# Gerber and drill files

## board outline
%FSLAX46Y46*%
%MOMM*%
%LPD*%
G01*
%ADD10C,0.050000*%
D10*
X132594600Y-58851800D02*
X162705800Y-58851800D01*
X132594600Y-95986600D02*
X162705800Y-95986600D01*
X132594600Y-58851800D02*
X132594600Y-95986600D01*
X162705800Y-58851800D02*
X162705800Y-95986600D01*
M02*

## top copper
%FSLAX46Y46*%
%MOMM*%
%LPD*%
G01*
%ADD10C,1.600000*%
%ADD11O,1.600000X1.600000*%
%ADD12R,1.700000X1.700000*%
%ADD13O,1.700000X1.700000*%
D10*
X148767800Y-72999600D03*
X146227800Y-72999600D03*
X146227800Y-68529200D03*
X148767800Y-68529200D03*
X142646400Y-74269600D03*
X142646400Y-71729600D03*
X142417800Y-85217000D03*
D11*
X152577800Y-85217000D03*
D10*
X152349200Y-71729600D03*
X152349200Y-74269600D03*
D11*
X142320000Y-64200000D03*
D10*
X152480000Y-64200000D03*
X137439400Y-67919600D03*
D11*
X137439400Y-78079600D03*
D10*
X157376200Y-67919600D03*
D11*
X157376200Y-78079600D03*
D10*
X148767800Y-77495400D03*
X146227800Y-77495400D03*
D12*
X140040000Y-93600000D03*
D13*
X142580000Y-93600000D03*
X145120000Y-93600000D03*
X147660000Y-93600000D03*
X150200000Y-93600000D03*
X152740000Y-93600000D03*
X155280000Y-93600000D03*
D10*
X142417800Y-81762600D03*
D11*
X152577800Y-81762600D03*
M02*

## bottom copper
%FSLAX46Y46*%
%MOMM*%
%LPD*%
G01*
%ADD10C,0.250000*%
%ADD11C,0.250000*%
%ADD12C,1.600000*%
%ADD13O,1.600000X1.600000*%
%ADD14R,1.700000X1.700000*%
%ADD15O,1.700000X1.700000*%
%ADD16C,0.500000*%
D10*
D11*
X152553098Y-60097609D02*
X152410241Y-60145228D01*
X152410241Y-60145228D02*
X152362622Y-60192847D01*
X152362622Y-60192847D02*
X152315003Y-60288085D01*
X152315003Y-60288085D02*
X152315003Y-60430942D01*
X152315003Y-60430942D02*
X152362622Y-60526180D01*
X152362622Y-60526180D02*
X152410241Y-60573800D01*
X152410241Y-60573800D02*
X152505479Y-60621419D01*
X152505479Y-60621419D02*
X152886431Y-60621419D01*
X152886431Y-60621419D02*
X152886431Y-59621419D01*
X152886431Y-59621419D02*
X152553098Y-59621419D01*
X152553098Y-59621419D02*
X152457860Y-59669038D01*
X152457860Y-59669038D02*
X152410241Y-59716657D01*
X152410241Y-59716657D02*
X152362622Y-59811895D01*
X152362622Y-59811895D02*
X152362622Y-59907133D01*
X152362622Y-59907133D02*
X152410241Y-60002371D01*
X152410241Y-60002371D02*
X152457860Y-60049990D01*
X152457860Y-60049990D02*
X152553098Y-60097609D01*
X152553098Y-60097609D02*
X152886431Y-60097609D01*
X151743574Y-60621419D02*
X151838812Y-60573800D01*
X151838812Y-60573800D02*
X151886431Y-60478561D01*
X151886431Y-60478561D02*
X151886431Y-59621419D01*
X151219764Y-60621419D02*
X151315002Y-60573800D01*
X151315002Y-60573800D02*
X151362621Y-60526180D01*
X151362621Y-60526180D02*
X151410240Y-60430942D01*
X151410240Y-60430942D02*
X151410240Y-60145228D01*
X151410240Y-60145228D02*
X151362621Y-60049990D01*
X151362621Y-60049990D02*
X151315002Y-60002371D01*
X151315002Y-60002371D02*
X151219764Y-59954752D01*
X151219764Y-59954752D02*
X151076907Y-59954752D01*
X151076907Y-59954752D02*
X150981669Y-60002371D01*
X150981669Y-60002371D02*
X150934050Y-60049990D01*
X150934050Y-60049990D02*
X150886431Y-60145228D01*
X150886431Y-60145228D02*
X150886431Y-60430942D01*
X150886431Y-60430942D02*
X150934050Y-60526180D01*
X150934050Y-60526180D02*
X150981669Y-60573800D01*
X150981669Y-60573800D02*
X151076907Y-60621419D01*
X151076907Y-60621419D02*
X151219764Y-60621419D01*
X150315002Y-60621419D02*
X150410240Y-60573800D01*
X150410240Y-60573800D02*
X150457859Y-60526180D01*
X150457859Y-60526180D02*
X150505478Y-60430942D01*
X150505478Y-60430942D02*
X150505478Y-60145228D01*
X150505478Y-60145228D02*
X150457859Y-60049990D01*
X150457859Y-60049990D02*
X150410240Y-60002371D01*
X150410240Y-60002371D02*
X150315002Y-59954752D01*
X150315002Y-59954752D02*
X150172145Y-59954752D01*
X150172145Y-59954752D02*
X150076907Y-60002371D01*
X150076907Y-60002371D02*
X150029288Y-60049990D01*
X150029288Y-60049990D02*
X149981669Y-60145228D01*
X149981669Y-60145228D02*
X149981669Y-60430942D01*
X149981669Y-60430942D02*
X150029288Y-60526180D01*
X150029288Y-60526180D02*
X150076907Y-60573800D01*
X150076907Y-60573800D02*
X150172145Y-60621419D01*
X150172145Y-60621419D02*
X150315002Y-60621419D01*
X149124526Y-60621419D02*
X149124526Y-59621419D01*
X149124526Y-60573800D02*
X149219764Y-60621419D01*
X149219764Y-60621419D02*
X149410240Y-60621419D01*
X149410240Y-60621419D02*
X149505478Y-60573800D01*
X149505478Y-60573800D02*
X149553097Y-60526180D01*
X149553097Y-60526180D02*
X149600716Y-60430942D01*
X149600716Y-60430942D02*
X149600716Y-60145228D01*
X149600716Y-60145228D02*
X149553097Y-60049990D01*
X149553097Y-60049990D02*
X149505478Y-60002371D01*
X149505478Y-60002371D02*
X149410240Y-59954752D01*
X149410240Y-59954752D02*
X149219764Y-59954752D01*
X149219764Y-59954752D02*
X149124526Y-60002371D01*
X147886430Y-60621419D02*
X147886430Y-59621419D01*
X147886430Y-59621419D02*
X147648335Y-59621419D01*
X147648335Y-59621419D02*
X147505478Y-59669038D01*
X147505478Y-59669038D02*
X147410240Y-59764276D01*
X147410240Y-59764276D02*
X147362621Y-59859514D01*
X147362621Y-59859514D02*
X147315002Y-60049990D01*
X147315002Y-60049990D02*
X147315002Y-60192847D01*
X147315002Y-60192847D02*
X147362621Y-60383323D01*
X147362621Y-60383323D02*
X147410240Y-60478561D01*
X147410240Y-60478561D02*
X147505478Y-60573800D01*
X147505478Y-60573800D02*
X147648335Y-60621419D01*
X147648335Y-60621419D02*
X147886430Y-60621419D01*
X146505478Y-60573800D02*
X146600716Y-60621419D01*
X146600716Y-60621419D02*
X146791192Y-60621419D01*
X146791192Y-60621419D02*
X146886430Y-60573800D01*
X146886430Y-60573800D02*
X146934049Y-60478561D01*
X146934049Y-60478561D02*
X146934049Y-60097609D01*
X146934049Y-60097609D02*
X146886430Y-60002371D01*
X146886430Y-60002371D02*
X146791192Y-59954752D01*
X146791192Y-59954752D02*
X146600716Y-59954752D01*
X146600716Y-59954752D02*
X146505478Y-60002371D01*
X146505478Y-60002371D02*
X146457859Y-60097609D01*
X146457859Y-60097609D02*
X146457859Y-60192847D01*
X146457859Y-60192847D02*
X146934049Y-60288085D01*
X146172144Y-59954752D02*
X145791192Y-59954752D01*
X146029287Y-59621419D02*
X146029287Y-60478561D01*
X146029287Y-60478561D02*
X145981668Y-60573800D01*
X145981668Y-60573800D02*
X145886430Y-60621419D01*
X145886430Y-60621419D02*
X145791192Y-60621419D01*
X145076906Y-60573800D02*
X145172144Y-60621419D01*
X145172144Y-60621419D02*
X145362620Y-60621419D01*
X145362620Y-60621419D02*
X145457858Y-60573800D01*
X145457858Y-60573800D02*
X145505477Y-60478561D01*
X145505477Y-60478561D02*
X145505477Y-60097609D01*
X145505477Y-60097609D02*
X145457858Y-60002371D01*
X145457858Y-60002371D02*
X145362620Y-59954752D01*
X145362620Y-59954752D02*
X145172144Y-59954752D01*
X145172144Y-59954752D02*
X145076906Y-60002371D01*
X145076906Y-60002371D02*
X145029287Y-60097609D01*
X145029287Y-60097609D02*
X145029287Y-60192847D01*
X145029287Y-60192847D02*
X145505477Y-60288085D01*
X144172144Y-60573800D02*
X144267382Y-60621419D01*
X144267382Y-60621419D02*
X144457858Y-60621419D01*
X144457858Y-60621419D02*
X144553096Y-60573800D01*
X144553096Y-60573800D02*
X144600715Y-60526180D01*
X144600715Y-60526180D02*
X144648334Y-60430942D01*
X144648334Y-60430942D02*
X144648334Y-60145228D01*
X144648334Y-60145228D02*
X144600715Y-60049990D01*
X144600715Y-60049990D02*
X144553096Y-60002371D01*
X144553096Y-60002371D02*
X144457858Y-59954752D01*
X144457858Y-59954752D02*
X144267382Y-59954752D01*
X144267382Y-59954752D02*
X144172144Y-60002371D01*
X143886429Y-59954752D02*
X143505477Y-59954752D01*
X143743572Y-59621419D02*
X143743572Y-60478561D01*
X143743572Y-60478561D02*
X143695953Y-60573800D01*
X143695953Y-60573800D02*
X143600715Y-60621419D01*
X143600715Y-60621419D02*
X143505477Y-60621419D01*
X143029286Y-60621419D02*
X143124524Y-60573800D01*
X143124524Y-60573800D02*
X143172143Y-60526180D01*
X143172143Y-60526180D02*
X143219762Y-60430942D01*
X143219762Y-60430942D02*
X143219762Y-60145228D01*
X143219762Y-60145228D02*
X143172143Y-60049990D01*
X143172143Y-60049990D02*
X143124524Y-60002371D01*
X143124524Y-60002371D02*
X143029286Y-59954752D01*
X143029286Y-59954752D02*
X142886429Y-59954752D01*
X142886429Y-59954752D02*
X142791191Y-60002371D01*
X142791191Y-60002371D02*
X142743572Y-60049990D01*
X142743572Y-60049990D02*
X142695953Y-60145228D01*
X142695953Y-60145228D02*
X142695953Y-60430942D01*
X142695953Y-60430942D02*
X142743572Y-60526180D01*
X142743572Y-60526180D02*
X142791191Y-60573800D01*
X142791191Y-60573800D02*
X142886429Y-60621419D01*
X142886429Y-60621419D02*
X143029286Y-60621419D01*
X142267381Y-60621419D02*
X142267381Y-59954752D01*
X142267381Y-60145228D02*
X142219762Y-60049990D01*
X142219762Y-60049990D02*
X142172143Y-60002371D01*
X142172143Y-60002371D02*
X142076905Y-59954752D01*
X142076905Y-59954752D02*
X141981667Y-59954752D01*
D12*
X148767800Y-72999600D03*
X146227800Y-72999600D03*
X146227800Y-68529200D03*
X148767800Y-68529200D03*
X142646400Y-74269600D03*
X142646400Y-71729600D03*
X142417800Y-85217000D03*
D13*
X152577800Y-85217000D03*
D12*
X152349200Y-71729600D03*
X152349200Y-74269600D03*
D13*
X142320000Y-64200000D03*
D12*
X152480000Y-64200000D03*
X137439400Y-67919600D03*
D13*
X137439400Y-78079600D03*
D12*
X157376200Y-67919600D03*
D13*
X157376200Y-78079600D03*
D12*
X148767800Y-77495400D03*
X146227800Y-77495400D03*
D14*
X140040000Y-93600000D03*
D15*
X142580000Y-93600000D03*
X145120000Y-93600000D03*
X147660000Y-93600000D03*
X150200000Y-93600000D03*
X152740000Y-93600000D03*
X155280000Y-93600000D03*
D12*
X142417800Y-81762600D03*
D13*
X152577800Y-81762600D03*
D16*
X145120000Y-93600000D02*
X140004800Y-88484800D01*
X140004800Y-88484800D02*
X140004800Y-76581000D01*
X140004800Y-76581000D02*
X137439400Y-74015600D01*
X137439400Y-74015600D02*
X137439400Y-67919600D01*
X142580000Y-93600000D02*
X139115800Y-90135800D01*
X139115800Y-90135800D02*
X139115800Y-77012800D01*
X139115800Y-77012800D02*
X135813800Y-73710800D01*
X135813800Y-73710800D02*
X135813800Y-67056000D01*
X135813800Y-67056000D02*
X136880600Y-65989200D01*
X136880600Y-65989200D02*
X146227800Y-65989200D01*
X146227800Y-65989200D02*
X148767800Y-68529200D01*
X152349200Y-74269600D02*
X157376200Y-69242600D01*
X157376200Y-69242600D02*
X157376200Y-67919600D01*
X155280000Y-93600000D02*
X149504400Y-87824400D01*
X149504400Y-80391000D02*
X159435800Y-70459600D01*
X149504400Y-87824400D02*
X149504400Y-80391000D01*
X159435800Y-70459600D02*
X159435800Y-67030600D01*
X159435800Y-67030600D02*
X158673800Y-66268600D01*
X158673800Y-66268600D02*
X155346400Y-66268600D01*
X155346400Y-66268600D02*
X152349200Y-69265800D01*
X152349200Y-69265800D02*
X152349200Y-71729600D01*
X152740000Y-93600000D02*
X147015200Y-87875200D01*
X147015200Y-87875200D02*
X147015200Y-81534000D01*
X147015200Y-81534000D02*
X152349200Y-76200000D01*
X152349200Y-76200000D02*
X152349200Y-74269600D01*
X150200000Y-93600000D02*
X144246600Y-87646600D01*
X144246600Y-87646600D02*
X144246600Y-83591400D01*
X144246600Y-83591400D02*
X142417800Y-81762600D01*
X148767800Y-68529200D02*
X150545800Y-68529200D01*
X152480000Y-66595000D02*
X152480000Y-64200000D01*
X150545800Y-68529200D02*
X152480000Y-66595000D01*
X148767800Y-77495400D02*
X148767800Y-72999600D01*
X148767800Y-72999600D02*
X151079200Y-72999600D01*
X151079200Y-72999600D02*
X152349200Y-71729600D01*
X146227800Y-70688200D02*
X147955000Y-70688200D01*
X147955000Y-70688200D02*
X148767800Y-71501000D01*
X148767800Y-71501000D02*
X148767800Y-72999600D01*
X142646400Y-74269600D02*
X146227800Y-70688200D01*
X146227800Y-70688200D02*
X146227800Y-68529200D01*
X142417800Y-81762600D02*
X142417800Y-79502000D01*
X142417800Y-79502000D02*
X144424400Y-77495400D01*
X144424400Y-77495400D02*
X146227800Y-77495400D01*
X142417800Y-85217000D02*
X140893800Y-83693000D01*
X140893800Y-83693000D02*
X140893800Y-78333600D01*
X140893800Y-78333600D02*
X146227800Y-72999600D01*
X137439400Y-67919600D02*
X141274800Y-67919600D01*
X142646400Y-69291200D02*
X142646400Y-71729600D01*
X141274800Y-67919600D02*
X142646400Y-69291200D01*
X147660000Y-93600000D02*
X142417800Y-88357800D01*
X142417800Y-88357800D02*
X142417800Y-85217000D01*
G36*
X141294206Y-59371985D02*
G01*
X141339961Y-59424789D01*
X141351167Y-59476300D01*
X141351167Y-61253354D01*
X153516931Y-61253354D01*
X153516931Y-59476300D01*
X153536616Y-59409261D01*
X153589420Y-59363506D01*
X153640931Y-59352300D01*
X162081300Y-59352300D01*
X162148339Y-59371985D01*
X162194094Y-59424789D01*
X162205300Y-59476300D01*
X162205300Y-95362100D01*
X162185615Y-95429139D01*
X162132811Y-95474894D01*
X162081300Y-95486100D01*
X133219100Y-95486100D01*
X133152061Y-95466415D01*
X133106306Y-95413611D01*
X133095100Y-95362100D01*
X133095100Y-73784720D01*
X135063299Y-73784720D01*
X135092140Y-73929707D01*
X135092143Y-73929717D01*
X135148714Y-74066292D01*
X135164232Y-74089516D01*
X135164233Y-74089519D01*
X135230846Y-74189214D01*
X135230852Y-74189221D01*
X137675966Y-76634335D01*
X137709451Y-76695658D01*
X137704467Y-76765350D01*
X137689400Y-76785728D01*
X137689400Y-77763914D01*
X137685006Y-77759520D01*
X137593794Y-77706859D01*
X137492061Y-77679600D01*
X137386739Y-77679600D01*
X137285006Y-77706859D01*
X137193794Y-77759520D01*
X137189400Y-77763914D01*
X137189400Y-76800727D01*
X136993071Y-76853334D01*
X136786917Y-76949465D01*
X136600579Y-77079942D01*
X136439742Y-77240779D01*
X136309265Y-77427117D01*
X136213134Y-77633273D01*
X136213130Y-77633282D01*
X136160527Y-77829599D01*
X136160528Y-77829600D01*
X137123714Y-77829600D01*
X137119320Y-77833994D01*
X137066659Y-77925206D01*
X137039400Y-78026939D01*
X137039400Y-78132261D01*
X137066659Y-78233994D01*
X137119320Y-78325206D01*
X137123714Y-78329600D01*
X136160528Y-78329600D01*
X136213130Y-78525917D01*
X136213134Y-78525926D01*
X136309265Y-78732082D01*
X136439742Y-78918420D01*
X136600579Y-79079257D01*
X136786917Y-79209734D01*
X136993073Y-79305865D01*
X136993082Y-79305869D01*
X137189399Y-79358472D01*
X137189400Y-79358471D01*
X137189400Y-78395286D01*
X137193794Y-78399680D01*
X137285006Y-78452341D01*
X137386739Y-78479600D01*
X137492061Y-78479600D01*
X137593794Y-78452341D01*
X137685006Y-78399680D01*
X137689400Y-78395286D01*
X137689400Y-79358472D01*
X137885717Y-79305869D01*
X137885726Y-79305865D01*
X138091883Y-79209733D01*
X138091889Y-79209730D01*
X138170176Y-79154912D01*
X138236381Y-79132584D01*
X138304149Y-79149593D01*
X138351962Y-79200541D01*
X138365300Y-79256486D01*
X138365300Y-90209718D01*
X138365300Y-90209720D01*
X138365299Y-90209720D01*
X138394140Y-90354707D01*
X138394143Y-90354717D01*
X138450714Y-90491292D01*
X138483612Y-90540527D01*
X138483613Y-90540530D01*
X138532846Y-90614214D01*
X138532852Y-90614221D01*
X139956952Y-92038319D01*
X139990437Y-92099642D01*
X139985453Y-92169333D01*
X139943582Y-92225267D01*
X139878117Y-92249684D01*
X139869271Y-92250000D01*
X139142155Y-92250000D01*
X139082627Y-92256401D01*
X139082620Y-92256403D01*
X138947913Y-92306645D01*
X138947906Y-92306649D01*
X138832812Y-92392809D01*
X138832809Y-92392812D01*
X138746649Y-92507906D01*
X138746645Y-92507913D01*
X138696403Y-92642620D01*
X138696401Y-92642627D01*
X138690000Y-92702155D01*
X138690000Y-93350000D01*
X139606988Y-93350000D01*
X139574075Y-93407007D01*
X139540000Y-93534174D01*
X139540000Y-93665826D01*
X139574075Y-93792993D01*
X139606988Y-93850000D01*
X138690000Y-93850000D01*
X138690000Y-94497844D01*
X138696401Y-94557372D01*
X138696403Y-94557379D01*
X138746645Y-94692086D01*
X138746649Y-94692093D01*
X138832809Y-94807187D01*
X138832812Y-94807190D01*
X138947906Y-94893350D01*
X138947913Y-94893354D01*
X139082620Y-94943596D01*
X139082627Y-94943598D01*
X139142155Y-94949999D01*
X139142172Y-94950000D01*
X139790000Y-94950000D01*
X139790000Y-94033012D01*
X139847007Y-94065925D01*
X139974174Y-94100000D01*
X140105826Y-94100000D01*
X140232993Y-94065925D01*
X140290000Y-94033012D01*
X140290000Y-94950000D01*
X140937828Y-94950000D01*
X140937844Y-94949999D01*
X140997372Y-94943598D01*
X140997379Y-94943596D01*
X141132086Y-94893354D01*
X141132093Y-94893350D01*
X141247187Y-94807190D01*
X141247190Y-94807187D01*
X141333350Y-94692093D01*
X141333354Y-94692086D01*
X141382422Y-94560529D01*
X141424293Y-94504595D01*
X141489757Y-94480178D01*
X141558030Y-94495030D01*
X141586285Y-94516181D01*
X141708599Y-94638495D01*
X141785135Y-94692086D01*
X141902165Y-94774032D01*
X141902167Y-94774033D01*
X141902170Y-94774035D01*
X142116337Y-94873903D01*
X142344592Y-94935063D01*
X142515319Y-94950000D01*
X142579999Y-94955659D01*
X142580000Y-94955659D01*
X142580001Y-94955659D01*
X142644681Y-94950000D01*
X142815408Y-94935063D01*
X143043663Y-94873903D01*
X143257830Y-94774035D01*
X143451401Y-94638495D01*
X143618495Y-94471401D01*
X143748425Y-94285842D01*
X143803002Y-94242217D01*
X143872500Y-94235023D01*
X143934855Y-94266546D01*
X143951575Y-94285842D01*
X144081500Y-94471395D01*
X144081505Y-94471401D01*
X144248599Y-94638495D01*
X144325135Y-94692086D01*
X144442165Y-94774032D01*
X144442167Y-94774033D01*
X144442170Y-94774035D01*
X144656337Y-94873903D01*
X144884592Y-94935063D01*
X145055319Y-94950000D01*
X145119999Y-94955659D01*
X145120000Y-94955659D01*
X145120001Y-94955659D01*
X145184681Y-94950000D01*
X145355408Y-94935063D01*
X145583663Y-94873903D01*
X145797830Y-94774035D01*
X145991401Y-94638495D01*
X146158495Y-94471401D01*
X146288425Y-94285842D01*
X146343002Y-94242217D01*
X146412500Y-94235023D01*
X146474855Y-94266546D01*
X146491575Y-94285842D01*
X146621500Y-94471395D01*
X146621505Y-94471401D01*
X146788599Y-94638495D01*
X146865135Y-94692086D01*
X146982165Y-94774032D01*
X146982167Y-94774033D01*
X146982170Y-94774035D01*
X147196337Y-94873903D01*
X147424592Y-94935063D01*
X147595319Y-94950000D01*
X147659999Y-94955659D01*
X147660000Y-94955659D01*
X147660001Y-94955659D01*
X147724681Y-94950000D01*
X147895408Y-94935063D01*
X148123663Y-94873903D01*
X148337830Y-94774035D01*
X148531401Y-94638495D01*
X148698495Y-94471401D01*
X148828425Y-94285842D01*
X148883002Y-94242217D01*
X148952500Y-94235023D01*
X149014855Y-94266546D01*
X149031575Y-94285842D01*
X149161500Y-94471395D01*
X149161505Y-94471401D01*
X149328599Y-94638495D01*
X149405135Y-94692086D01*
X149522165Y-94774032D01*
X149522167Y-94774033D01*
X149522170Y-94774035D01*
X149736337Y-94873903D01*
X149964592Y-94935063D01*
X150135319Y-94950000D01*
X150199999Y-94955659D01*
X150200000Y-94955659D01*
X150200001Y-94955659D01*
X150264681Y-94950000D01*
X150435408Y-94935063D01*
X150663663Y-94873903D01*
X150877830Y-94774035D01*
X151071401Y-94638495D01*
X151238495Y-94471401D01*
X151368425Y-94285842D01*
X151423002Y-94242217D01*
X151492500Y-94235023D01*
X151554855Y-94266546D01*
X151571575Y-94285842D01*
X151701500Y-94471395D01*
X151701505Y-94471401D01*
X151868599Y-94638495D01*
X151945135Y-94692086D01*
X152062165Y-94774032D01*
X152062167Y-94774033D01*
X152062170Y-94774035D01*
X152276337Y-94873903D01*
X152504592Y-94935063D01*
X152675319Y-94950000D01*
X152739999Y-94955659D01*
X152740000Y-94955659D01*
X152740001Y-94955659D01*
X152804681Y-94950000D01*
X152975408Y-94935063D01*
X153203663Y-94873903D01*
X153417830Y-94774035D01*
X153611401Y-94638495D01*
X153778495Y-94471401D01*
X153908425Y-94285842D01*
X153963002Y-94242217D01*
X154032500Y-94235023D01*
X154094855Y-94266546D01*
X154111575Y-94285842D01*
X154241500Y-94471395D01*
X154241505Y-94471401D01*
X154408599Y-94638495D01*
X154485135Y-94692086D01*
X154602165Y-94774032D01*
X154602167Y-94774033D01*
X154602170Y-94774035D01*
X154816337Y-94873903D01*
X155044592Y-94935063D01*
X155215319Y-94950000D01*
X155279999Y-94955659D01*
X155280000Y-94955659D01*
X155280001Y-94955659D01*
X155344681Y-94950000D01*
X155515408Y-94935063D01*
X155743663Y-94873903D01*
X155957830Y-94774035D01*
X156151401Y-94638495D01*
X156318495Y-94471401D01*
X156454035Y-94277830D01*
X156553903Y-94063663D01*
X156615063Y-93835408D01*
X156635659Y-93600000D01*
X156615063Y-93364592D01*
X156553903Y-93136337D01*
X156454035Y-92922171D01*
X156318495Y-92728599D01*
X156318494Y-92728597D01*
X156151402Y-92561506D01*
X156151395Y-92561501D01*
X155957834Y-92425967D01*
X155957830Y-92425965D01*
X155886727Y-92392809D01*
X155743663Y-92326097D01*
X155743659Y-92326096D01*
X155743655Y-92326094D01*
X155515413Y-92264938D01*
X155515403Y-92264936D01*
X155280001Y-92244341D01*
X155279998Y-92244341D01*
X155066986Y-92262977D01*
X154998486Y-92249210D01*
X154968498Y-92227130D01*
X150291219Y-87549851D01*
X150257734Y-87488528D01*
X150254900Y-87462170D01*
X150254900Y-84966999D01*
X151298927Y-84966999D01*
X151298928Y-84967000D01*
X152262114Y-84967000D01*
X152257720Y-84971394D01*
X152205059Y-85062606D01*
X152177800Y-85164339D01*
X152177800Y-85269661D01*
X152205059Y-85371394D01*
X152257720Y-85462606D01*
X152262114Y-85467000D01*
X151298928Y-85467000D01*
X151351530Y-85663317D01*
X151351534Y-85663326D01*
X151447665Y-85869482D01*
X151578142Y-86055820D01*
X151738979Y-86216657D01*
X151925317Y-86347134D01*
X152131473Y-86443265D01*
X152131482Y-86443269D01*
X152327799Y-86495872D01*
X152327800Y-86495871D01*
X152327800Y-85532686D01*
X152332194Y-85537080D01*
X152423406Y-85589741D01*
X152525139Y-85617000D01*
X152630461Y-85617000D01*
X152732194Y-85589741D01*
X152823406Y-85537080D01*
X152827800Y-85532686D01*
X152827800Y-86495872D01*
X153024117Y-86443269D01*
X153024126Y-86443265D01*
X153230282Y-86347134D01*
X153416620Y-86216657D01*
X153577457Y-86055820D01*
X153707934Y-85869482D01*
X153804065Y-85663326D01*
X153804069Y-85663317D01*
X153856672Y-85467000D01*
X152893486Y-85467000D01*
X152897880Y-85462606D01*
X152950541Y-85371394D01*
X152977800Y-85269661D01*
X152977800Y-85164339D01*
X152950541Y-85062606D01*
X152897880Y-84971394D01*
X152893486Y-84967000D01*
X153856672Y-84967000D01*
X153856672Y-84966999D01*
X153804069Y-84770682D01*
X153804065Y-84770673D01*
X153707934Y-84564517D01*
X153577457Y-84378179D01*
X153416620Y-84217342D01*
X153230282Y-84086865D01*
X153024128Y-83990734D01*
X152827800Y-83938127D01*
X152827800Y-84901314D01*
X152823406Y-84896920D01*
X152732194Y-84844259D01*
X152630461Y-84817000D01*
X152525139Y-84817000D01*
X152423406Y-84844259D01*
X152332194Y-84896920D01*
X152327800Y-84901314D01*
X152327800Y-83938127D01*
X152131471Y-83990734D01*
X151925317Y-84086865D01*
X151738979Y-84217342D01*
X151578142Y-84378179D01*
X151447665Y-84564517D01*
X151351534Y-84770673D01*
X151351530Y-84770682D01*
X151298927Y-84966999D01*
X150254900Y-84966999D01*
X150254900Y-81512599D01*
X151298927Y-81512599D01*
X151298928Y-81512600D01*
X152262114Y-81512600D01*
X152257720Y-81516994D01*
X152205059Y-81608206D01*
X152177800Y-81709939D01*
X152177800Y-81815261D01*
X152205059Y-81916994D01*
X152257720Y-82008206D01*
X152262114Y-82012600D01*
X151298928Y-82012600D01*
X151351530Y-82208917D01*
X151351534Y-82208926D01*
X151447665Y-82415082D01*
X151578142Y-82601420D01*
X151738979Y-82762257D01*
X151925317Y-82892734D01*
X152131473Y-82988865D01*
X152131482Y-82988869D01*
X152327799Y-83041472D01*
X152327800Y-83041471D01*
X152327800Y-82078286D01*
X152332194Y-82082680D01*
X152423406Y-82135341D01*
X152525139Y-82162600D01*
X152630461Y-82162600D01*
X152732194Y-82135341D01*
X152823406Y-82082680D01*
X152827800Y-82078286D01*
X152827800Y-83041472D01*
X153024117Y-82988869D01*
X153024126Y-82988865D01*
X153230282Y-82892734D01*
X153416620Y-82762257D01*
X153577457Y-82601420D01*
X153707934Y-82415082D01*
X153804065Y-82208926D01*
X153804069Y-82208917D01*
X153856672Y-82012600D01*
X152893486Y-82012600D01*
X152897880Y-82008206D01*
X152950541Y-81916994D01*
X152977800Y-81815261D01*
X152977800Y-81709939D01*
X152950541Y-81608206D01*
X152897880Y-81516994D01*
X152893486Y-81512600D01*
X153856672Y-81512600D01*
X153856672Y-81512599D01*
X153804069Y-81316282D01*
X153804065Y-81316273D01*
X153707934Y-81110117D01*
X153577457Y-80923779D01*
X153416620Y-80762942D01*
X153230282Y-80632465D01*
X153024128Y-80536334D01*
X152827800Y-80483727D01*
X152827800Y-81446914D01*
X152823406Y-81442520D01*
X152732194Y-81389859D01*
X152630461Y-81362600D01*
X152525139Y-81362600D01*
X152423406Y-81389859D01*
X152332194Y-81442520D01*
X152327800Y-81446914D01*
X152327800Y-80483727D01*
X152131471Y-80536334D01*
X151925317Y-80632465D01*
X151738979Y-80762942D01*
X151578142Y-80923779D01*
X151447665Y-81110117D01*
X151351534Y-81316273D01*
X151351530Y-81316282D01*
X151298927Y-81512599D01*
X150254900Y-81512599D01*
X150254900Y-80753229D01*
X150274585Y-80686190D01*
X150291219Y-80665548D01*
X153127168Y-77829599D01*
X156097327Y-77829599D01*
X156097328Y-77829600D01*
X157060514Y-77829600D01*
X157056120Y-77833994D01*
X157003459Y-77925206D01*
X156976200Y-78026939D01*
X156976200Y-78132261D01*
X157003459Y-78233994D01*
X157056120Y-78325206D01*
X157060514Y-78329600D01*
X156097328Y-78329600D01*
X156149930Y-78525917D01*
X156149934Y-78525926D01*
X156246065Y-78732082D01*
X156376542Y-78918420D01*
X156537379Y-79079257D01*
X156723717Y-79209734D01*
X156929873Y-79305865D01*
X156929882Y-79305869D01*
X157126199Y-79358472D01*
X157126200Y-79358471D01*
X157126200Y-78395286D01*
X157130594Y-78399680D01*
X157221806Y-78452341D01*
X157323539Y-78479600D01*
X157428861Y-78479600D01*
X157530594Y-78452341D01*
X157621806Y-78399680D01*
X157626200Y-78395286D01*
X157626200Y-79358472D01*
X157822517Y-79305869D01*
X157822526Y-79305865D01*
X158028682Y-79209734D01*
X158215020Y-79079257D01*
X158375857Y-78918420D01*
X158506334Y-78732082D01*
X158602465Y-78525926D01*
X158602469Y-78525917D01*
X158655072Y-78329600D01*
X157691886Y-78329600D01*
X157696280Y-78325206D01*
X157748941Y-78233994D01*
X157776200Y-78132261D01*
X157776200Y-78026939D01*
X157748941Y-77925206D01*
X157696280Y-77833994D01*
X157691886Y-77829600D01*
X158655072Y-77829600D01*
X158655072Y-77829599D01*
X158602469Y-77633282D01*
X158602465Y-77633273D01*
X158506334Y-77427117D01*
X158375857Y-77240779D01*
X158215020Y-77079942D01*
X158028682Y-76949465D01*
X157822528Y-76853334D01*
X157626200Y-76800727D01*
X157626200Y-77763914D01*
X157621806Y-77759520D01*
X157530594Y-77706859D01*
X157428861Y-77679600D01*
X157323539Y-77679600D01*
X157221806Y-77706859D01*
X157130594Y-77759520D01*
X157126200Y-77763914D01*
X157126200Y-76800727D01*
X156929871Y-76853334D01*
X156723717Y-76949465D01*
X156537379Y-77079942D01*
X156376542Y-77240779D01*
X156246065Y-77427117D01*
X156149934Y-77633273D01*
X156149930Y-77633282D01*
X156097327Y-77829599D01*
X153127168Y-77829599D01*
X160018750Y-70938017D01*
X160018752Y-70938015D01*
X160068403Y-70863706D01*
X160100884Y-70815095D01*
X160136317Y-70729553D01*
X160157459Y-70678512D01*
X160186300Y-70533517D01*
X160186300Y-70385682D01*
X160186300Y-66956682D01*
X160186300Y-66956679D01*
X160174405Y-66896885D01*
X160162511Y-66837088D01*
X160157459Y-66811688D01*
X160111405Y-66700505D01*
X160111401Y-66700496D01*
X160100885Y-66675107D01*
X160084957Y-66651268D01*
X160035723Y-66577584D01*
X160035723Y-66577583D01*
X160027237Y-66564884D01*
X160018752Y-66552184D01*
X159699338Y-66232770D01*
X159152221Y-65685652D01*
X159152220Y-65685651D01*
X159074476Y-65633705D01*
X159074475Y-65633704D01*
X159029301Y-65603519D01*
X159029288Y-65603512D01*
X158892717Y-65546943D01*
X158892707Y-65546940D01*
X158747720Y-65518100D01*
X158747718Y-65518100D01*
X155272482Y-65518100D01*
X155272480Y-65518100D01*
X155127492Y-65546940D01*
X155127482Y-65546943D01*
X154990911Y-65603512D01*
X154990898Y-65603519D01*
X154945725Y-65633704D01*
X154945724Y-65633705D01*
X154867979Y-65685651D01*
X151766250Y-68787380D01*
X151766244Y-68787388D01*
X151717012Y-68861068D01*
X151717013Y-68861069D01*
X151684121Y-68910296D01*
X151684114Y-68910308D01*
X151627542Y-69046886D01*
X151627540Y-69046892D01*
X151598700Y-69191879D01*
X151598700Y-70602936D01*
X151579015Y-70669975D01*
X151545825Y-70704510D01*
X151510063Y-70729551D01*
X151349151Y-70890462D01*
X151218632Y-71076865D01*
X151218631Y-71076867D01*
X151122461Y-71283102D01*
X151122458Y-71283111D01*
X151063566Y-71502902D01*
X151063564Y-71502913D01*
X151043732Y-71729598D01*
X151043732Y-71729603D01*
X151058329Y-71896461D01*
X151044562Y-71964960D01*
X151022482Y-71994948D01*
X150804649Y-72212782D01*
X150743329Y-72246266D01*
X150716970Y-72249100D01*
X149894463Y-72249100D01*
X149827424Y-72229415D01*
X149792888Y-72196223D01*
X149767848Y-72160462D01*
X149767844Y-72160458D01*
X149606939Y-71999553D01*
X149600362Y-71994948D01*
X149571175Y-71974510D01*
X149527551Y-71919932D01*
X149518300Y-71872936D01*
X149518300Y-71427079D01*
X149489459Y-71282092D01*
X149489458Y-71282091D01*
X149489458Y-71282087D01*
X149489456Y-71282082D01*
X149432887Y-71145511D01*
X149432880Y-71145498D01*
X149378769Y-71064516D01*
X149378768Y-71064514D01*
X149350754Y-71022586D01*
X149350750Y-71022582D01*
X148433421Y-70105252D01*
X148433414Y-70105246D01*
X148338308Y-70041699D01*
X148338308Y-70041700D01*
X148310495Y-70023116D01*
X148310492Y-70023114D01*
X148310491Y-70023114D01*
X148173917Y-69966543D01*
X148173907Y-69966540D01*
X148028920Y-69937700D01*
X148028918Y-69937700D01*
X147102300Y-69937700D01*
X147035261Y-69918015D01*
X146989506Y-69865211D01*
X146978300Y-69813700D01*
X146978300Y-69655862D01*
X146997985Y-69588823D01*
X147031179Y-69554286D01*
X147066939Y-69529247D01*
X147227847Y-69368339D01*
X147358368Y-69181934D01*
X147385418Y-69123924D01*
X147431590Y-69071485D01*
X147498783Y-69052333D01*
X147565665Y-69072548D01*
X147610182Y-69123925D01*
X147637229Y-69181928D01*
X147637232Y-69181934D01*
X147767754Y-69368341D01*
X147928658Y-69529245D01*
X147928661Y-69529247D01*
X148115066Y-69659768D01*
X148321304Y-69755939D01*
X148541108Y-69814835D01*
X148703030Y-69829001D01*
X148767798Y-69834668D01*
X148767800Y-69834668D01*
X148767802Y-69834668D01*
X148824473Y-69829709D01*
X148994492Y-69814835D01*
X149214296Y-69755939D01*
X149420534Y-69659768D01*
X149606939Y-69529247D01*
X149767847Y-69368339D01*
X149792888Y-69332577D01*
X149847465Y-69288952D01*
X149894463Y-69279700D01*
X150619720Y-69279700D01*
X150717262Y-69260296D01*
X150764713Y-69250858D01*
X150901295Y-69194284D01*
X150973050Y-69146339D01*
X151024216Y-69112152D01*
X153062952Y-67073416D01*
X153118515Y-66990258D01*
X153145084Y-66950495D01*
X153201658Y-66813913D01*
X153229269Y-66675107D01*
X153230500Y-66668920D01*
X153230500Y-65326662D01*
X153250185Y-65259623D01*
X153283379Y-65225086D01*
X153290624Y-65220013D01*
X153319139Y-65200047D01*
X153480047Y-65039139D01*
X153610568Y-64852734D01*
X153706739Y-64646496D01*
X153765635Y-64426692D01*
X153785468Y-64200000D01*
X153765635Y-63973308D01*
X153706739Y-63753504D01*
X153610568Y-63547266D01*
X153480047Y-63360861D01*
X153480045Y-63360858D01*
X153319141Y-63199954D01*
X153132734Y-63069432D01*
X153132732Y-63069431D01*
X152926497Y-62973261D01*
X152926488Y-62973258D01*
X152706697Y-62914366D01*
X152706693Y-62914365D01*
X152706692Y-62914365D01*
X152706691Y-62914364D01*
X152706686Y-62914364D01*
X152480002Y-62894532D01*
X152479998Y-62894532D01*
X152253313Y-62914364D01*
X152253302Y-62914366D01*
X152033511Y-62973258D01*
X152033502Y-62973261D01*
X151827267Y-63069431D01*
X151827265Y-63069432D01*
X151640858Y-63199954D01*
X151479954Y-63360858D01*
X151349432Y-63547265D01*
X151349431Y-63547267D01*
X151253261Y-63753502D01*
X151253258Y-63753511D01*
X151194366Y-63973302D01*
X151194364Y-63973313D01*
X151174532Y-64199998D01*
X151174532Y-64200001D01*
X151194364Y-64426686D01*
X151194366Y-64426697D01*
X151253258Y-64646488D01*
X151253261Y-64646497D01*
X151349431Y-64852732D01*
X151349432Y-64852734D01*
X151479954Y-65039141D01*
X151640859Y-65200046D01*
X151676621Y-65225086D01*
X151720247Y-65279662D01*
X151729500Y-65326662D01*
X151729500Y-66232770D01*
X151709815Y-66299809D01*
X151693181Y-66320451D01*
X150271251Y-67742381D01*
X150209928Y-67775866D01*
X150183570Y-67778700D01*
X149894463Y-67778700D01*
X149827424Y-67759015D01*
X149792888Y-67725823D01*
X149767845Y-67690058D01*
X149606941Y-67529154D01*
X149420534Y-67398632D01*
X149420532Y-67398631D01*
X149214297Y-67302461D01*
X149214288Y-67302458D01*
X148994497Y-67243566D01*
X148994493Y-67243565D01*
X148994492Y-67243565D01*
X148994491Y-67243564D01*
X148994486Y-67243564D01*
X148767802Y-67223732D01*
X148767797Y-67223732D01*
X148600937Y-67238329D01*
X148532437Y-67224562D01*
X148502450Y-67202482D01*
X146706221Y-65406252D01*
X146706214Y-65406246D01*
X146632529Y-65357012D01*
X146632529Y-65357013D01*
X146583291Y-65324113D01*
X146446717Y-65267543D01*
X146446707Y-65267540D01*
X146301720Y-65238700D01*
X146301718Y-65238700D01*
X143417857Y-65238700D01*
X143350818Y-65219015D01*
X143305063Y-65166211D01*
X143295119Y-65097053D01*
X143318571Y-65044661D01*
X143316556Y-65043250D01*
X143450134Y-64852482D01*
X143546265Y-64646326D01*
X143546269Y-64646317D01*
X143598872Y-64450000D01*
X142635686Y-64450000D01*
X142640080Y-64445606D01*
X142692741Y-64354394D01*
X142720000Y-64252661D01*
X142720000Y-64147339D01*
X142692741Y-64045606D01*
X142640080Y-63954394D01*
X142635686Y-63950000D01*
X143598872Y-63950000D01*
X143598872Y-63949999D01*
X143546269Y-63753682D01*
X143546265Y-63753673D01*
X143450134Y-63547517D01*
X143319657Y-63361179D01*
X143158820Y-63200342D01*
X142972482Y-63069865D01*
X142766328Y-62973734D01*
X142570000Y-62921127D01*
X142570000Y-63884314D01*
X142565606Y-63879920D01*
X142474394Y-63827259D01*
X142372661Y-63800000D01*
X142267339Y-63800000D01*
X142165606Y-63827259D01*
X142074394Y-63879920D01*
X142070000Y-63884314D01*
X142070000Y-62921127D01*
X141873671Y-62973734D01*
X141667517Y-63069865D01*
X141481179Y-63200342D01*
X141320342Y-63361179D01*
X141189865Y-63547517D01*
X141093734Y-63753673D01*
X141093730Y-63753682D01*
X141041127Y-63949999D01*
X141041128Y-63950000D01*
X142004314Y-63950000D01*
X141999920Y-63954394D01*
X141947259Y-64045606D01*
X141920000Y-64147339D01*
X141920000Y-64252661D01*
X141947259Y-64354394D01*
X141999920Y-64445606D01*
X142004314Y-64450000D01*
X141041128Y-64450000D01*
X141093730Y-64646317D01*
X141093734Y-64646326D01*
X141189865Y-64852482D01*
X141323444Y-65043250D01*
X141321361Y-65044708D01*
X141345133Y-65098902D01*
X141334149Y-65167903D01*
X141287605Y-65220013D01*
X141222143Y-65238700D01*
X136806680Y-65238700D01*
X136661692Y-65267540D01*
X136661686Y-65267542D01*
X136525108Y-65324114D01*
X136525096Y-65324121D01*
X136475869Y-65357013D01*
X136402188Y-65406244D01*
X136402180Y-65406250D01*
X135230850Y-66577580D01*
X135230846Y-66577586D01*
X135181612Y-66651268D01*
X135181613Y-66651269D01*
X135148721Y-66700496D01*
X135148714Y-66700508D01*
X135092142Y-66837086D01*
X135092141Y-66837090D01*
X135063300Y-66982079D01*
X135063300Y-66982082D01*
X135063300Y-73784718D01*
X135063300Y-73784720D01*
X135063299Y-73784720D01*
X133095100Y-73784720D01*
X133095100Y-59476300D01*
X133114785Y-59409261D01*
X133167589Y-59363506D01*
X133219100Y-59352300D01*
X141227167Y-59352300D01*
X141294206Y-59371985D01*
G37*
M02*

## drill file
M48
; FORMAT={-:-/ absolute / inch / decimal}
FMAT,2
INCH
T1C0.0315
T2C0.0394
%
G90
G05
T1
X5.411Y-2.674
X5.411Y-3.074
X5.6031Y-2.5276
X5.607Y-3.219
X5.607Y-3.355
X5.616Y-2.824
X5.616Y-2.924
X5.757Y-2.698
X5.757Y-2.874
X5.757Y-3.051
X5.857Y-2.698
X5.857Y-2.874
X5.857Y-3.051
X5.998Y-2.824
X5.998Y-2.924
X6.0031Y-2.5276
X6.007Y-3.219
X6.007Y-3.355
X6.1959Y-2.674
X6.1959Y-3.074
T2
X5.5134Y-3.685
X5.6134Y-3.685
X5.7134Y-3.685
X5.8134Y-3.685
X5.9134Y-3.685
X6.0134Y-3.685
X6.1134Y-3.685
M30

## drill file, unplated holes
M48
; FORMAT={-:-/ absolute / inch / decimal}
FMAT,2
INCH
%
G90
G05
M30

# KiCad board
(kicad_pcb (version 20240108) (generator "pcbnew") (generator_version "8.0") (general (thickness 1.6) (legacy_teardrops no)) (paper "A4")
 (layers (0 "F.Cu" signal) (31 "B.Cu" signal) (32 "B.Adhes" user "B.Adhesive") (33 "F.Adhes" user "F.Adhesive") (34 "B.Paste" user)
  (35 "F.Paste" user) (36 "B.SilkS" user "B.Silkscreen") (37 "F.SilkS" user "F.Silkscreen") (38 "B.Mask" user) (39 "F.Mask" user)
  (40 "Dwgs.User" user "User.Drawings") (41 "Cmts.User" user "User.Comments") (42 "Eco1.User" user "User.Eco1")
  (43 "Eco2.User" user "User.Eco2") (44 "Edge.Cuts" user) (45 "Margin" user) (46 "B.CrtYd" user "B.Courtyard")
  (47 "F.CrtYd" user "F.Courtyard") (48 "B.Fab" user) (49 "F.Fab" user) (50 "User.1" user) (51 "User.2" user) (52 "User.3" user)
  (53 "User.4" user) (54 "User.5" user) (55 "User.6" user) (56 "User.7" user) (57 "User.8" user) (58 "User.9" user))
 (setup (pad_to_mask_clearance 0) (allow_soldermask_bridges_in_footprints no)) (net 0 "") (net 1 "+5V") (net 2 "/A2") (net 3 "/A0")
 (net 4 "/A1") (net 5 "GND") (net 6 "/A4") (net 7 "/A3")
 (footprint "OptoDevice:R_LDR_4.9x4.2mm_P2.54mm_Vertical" (layer "F.Cu") (at 148.7678 72.9996 180)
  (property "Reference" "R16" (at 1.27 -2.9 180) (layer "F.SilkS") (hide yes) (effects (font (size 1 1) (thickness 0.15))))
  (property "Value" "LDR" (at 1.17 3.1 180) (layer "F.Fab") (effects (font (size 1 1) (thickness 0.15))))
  (pad "1" thru_hole circle (at 0 0 180) (size 1.6 1.6) (drill 0.8) (layers "*.Cu" "*.Mask") (remove_unused_layers no) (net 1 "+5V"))
  (pad "2" thru_hole circle (at 2.54 0 180) (size 1.6 1.6) (drill 0.8) (layers "*.Cu" "*.Mask") (remove_unused_layers no) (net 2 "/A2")))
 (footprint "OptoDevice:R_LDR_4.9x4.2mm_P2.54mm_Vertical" (layer "F.Cu") (at 146.2278 68.5292)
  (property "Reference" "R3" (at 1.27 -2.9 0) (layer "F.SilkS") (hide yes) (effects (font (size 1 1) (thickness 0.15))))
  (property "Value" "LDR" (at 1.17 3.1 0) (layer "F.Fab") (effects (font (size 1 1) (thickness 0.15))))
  (pad "1" thru_hole circle (at 0 0) (size 1.6 1.6) (drill 0.8) (layers "*.Cu" "*.Mask") (remove_unused_layers no) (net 1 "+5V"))
  (pad "2" thru_hole circle (at 2.54 0) (size 1.6 1.6) (drill 0.8) (layers "*.Cu" "*.Mask") (remove_unused_layers no) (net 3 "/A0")))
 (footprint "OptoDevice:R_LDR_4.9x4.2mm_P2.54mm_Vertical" (layer "F.Cu") (at 142.6464 74.2696 90)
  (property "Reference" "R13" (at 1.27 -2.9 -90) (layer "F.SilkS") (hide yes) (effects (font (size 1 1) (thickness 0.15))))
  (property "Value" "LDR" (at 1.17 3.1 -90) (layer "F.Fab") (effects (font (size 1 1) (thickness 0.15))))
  (pad "1" thru_hole circle (at 0 0 90) (size 1.6 1.6) (drill 0.8) (layers "*.Cu" "*.Mask") (remove_unused_layers no) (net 1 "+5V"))
  (pad "2" thru_hole circle (at 2.54 0 90) (size 1.6 1.6) (drill 0.8) (layers "*.Cu" "*.Mask") (remove_unused_layers no) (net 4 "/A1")))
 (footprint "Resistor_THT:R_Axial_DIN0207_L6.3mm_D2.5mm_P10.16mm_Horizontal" (layer "F.Cu") (at 142.4178 85.217)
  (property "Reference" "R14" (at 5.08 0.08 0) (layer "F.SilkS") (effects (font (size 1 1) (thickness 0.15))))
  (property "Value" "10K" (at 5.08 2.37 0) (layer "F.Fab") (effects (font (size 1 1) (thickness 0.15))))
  (pad "1" thru_hole circle (at 0 0) (size 1.6 1.6) (drill 0.8) (layers "*.Cu" "*.Mask") (remove_unused_layers no) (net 2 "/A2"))
  (pad "2" thru_hole oval (at 10.16 0) (size 1.6 1.6) (drill 0.8) (layers "*.Cu" "*.Mask") (remove_unused_layers no) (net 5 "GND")))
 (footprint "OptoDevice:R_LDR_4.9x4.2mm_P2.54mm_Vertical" (layer "F.Cu") (at 152.3492 71.7296 -90)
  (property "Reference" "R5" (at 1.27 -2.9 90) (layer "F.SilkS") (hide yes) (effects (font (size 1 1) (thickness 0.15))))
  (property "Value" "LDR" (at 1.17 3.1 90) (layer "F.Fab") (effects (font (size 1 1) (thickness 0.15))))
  (pad "1" thru_hole circle (at 0 0 270) (size 1.6 1.6) (drill 0.8) (layers "*.Cu" "*.Mask") (remove_unused_layers no) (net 1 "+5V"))
  (pad "2" thru_hole circle (at 2.54 0 270) (size 1.6 1.6) (drill 0.8) (layers "*.Cu" "*.Mask") (remove_unused_layers no) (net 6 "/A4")))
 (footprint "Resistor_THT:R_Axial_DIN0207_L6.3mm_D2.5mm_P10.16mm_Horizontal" (layer "F.Cu") (at 152.48 64.2 180)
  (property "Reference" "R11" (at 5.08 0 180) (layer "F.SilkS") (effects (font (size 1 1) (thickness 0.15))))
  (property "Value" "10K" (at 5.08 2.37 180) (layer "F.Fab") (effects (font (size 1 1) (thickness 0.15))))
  (pad "1" thru_hole circle (at 0 0 180) (size 1.6 1.6) (drill 0.8) (layers "*.Cu" "*.Mask") (remove_unused_layers no) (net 3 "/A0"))
  (pad "2" thru_hole oval (at 10.16 0 180) (size 1.6 1.6) (drill 0.8) (layers "*.Cu" "*.Mask") (remove_unused_layers no) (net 5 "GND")))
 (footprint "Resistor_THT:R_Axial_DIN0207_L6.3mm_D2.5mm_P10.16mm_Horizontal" (layer "F.Cu") (at 137.4394 67.9196 -90)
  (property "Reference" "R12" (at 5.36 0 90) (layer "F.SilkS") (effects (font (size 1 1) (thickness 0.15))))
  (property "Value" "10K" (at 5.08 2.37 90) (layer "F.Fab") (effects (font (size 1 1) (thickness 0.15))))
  (pad "1" thru_hole circle (at 0 0 270) (size 1.6 1.6) (drill 0.8) (layers "*.Cu" "*.Mask") (remove_unused_layers no) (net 4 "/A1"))
  (pad "2" thru_hole oval (at 10.16 0 270) (size 1.6 1.6) (drill 0.8) (layers "*.Cu" "*.Mask") (remove_unused_layers no) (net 5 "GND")))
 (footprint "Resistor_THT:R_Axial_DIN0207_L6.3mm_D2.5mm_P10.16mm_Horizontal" (layer "F.Cu") (at 157.3762 67.9196 -90)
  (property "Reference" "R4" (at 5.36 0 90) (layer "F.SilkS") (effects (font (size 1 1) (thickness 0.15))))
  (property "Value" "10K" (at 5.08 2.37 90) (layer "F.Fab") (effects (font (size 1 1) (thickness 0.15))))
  (pad "1" thru_hole circle (at 0 0 270) (size 1.6 1.6) (drill 0.8) (layers "*.Cu" "*.Mask") (remove_unused_layers no) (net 6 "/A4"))
  (pad "2" thru_hole oval (at 10.16 0 270) (size 1.6 1.6) (drill 0.8) (layers "*.Cu" "*.Mask") (remove_unused_layers no) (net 5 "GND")))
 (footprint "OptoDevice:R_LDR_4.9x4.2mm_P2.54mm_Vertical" (layer "F.Cu") (at 148.7678 77.4954 180)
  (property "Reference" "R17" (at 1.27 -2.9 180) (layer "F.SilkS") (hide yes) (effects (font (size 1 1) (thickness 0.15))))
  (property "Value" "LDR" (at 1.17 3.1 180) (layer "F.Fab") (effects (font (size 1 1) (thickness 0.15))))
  (pad "1" thru_hole circle (at 0 0 180) (size 1.6 1.6) (drill 0.8) (layers "*.Cu" "*.Mask") (remove_unused_layers no) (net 1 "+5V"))
  (pad "2" thru_hole circle (at 2.54 0 180) (size 1.6 1.6) (drill 0.8) (layers "*.Cu" "*.Mask") (remove_unused_layers no) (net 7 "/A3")))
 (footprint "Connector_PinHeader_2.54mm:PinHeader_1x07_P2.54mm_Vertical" (layer "F.Cu") (at 140.04 93.6 90)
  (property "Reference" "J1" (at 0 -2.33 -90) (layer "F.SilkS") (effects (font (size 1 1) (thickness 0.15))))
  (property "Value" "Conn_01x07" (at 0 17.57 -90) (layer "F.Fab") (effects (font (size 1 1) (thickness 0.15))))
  (pad "1" thru_hole rect (at 0 0 90) (size 1.7 1.7) (drill 1) (layers "*.Cu" "*.Mask") (remove_unused_layers no) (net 5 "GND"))
  (pad "2" thru_hole oval (at 0 2.54 90) (size 1.7 1.7) (drill 1) (layers "*.Cu" "*.Mask") (remove_unused_layers no) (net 3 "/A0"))
  (pad "3" thru_hole oval (at 0 5.08 90) (size 1.7 1.7) (drill 1) (layers "*.Cu" "*.Mask") (remove_unused_layers no) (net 4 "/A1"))
  (pad "4" thru_hole oval (at 0 7.62 90) (size 1.7 1.7) (drill 1) (layers "*.Cu" "*.Mask") (remove_unused_layers no) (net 2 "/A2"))
  (pad "5" thru_hole oval (at 0 10.16 90) (size 1.7 1.7) (drill 1) (layers "*.Cu" "*.Mask") (remove_unused_layers no) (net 7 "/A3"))
  (pad "6" thru_hole oval (at 0 12.7 90) (size 1.7 1.7) (drill 1) (layers "*.Cu" "*.Mask") (remove_unused_layers no) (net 6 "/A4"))
  (pad "7" thru_hole oval (at 0 15.24 90) (size 1.7 1.7) (drill 1) (layers "*.Cu" "*.Mask") (remove_unused_layers no) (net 1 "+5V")))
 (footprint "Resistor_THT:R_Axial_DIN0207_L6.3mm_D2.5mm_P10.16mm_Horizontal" (layer "F.Cu") (at 142.4178 81.7626)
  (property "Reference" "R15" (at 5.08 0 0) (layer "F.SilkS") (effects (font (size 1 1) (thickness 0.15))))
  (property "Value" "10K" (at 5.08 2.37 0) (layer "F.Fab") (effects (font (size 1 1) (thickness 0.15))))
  (pad "1" thru_hole circle (at 0 0) (size 1.6 1.6) (drill 0.8) (layers "*.Cu" "*.Mask") (remove_unused_layers no) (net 7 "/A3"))
  (pad "2" thru_hole oval (at 10.16 0) (size 1.6 1.6) (drill 0.8) (layers "*.Cu" "*.Mask") (remove_unused_layers no) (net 5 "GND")))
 (gr_line (start 132.5946 58.8518) (end 162.7058 58.8518) (stroke (width 0.05) (type default)) (layer "Edge.Cuts"))
 (gr_line (start 132.5946 58.8518) (end 132.5946 95.9866) (stroke (width 0.05) (type default)) (layer "Edge.Cuts"))
 (gr_line (start 132.5946 95.9866) (end 162.7058 95.9866) (stroke (width 0.05) (type default)) (layer "Edge.Cuts"))
 (gr_line (start 162.7058 58.8518) (end 162.7058 95.9866) (stroke (width 0.05) (type default)) (layer "Edge.Cuts"))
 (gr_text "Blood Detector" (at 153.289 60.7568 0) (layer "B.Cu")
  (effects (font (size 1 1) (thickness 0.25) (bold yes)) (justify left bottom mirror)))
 (segment (start 158.6738 66.2686) (end 155.3464 66.2686) (width 0.5) (layer "B.Cu") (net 1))
 (segment (start 152.3492 69.2658) (end 152.3492 71.7296) (width 0.5) (layer "B.Cu") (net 1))
 (segment (start 159.4358 70.4596) (end 159.4358 67.0306) (width 0.5) (layer "B.Cu") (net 1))
 (segment (start 155.3464 66.2686) (end 152.3492 69.2658) (width 0.5) (layer "B.Cu") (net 1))
 (segment (start 149.5044 87.8244) (end 149.5044 80.391) (width 0.5) (layer "B.Cu") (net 1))
 (segment (start 146.2278 70.6882) (end 147.955 70.6882) (width 0.5) (layer "B.Cu") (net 1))
 (segment (start 142.6464 74.2696) (end 146.2278 70.6882) (width 0.5) (layer "B.Cu") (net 1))
 (segment (start 148.7678 71.501) (end 148.7678 72.9996) (width 0.5) (layer "B.Cu") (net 1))
 (segment (start 148.7678 77.4954) (end 148.7678 72.9996) (width 0.5) (layer "B.Cu") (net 1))
 (segment (start 155.28 93.6) (end 149.5044 87.8244) (width 0.5) (layer "B.Cu") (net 1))
 (segment (start 149.5044 80.391) (end 159.4358 70.4596) (width 0.5) (layer "B.Cu") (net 1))
 (segment (start 146.2278 70.6882) (end 146.2278 68.5292) (width 0.5) (layer "B.Cu") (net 1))
 (segment (start 147.955 70.6882) (end 148.7678 71.501) (width 0.5) (layer "B.Cu") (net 1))
 (segment (start 151.0792 72.9996) (end 152.3492 71.7296) (width 0.5) (layer "B.Cu") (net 1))
 (segment (start 148.7678 72.9996) (end 151.0792 72.9996) (width 0.5) (layer "B.Cu") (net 1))
 (segment (start 159.4358 67.0306) (end 158.6738 66.2686) (width 0.5) (layer "B.Cu") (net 1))
 (segment (start 135.8138 73.7108) (end 135.8138 67.056) (width 0.5) (layer "B.Cu") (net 3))
 (segment (start 148.7678 68.5292) (end 150.5458 68.5292) (width 0.5) (layer "B.Cu") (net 3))
 (segment (start 136.8806 65.9892) (end 146.2278 65.9892) (width 0.5) (layer "B.Cu") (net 3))
 (segment (start 142.58 93.6) (end 139.1158 90.1358) (width 0.5) (layer "B.Cu") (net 3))
 (segment (start 139.1158 90.1358) (end 139.1158 77.0128) (width 0.5) (layer "B.Cu") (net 3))
 (segment (start 146.2278 65.9892) (end 148.7678 68.5292) (width 0.5) (layer "B.Cu") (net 3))
 (segment (start 150.5458 68.5292) (end 152.48 66.595) (width 0.5) (layer "B.Cu") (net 3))
 (segment (start 139.1158 77.0128) (end 135.8138 73.7108) (width 0.5) (layer "B.Cu") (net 3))
 (segment (start 135.8138 67.056) (end 136.8806 65.9892) (width 0.5) (layer "B.Cu") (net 3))
 (segment (start 152.48 66.595) (end 152.48 64.2) (width 0.5) (layer "B.Cu") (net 3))
 (segment (start 147.0152 87.8752) (end 147.0152 81.534) (width 0.5) (layer "B.Cu") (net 6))
 (segment (start 152.74 93.6) (end 147.0152 87.8752) (width 0.5) (layer "B.Cu") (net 6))
 (segment (start 147.0152 81.534) (end 152.3492 76.2) (width 0.5) (layer "B.Cu") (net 6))
 (segment (start 157.3762 69.2426) (end 157.3762 67.9196) (width 0.5) (layer "B.Cu") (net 6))
 (segment (start 152.3492 76.2) (end 152.3492 74.2696) (width 0.5) (layer "B.Cu") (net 6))
 (segment (start 152.3492 74.2696) (end 157.3762 69.2426) (width 0.5) (layer "B.Cu") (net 6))
 (segment (start 137.4394 74.0156) (end 137.4394 67.9196) (width 0.5) (layer "B.Cu") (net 4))
 (segment (start 142.6464 69.2912) (end 142.6464 71.7296) (width 0.5) (layer "B.Cu") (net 4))
 (segment (start 141.2748 67.9196) (end 142.6464 69.2912) (width 0.5) (layer "B.Cu") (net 4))
 (segment (start 137.4394 67.9196) (end 141.2748 67.9196) (width 0.5) (layer "B.Cu") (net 4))
 (segment (start 145.12 93.6) (end 140.0048 88.4848) (width 0.5) (layer "B.Cu") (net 4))
 (segment (start 140.0048 88.4848) (end 140.0048 76.581) (width 0.5) (layer "B.Cu") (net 4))
 (segment (start 140.0048 76.581) (end 137.4394 74.0156) (width 0.5) (layer "B.Cu") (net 4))
 (segment (start 147.66 93.6) (end 142.4178 88.3578) (width 0.5) (layer "B.Cu") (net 2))
 (segment (start 142.4178 88.3578) (end 142.4178 85.217) (width 0.5) (layer "B.Cu") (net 2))
 (segment (start 140.8938 78.3336) (end 146.2278 72.9996) (width 0.5) (layer "B.Cu") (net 2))
 (segment (start 140.8938 83.693) (end 140.8938 78.3336) (width 0.5) (layer "B.Cu") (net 2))
 (segment (start 142.4178 85.217) (end 140.8938 83.693) (width 0.5) (layer "B.Cu") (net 2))
 (segment (start 144.4244 77.4954) (end 146.2278 77.4954) (width 0.5) (layer "B.Cu") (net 7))
 (segment (start 144.2466 87.6466) (end 144.2466 83.5914) (width 0.5) (layer "B.Cu") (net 7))
 (segment (start 142.4178 79.502) (end 144.4244 77.4954) (width 0.5) (layer "B.Cu") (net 7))
 (segment (start 144.2466 83.5914) (end 142.4178 81.7626) (width 0.5) (layer "B.Cu") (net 7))
 (segment (start 150.2 93.6) (end 144.2466 87.6466) (width 0.5) (layer "B.Cu") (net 7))
 (segment (start 142.4178 81.7626) (end 142.4178 79.502) (width 0.5) (layer "B.Cu") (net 7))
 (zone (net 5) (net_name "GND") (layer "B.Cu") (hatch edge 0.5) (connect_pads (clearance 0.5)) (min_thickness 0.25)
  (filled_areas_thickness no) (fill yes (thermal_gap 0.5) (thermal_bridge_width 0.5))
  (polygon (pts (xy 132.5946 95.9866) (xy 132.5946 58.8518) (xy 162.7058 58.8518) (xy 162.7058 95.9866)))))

